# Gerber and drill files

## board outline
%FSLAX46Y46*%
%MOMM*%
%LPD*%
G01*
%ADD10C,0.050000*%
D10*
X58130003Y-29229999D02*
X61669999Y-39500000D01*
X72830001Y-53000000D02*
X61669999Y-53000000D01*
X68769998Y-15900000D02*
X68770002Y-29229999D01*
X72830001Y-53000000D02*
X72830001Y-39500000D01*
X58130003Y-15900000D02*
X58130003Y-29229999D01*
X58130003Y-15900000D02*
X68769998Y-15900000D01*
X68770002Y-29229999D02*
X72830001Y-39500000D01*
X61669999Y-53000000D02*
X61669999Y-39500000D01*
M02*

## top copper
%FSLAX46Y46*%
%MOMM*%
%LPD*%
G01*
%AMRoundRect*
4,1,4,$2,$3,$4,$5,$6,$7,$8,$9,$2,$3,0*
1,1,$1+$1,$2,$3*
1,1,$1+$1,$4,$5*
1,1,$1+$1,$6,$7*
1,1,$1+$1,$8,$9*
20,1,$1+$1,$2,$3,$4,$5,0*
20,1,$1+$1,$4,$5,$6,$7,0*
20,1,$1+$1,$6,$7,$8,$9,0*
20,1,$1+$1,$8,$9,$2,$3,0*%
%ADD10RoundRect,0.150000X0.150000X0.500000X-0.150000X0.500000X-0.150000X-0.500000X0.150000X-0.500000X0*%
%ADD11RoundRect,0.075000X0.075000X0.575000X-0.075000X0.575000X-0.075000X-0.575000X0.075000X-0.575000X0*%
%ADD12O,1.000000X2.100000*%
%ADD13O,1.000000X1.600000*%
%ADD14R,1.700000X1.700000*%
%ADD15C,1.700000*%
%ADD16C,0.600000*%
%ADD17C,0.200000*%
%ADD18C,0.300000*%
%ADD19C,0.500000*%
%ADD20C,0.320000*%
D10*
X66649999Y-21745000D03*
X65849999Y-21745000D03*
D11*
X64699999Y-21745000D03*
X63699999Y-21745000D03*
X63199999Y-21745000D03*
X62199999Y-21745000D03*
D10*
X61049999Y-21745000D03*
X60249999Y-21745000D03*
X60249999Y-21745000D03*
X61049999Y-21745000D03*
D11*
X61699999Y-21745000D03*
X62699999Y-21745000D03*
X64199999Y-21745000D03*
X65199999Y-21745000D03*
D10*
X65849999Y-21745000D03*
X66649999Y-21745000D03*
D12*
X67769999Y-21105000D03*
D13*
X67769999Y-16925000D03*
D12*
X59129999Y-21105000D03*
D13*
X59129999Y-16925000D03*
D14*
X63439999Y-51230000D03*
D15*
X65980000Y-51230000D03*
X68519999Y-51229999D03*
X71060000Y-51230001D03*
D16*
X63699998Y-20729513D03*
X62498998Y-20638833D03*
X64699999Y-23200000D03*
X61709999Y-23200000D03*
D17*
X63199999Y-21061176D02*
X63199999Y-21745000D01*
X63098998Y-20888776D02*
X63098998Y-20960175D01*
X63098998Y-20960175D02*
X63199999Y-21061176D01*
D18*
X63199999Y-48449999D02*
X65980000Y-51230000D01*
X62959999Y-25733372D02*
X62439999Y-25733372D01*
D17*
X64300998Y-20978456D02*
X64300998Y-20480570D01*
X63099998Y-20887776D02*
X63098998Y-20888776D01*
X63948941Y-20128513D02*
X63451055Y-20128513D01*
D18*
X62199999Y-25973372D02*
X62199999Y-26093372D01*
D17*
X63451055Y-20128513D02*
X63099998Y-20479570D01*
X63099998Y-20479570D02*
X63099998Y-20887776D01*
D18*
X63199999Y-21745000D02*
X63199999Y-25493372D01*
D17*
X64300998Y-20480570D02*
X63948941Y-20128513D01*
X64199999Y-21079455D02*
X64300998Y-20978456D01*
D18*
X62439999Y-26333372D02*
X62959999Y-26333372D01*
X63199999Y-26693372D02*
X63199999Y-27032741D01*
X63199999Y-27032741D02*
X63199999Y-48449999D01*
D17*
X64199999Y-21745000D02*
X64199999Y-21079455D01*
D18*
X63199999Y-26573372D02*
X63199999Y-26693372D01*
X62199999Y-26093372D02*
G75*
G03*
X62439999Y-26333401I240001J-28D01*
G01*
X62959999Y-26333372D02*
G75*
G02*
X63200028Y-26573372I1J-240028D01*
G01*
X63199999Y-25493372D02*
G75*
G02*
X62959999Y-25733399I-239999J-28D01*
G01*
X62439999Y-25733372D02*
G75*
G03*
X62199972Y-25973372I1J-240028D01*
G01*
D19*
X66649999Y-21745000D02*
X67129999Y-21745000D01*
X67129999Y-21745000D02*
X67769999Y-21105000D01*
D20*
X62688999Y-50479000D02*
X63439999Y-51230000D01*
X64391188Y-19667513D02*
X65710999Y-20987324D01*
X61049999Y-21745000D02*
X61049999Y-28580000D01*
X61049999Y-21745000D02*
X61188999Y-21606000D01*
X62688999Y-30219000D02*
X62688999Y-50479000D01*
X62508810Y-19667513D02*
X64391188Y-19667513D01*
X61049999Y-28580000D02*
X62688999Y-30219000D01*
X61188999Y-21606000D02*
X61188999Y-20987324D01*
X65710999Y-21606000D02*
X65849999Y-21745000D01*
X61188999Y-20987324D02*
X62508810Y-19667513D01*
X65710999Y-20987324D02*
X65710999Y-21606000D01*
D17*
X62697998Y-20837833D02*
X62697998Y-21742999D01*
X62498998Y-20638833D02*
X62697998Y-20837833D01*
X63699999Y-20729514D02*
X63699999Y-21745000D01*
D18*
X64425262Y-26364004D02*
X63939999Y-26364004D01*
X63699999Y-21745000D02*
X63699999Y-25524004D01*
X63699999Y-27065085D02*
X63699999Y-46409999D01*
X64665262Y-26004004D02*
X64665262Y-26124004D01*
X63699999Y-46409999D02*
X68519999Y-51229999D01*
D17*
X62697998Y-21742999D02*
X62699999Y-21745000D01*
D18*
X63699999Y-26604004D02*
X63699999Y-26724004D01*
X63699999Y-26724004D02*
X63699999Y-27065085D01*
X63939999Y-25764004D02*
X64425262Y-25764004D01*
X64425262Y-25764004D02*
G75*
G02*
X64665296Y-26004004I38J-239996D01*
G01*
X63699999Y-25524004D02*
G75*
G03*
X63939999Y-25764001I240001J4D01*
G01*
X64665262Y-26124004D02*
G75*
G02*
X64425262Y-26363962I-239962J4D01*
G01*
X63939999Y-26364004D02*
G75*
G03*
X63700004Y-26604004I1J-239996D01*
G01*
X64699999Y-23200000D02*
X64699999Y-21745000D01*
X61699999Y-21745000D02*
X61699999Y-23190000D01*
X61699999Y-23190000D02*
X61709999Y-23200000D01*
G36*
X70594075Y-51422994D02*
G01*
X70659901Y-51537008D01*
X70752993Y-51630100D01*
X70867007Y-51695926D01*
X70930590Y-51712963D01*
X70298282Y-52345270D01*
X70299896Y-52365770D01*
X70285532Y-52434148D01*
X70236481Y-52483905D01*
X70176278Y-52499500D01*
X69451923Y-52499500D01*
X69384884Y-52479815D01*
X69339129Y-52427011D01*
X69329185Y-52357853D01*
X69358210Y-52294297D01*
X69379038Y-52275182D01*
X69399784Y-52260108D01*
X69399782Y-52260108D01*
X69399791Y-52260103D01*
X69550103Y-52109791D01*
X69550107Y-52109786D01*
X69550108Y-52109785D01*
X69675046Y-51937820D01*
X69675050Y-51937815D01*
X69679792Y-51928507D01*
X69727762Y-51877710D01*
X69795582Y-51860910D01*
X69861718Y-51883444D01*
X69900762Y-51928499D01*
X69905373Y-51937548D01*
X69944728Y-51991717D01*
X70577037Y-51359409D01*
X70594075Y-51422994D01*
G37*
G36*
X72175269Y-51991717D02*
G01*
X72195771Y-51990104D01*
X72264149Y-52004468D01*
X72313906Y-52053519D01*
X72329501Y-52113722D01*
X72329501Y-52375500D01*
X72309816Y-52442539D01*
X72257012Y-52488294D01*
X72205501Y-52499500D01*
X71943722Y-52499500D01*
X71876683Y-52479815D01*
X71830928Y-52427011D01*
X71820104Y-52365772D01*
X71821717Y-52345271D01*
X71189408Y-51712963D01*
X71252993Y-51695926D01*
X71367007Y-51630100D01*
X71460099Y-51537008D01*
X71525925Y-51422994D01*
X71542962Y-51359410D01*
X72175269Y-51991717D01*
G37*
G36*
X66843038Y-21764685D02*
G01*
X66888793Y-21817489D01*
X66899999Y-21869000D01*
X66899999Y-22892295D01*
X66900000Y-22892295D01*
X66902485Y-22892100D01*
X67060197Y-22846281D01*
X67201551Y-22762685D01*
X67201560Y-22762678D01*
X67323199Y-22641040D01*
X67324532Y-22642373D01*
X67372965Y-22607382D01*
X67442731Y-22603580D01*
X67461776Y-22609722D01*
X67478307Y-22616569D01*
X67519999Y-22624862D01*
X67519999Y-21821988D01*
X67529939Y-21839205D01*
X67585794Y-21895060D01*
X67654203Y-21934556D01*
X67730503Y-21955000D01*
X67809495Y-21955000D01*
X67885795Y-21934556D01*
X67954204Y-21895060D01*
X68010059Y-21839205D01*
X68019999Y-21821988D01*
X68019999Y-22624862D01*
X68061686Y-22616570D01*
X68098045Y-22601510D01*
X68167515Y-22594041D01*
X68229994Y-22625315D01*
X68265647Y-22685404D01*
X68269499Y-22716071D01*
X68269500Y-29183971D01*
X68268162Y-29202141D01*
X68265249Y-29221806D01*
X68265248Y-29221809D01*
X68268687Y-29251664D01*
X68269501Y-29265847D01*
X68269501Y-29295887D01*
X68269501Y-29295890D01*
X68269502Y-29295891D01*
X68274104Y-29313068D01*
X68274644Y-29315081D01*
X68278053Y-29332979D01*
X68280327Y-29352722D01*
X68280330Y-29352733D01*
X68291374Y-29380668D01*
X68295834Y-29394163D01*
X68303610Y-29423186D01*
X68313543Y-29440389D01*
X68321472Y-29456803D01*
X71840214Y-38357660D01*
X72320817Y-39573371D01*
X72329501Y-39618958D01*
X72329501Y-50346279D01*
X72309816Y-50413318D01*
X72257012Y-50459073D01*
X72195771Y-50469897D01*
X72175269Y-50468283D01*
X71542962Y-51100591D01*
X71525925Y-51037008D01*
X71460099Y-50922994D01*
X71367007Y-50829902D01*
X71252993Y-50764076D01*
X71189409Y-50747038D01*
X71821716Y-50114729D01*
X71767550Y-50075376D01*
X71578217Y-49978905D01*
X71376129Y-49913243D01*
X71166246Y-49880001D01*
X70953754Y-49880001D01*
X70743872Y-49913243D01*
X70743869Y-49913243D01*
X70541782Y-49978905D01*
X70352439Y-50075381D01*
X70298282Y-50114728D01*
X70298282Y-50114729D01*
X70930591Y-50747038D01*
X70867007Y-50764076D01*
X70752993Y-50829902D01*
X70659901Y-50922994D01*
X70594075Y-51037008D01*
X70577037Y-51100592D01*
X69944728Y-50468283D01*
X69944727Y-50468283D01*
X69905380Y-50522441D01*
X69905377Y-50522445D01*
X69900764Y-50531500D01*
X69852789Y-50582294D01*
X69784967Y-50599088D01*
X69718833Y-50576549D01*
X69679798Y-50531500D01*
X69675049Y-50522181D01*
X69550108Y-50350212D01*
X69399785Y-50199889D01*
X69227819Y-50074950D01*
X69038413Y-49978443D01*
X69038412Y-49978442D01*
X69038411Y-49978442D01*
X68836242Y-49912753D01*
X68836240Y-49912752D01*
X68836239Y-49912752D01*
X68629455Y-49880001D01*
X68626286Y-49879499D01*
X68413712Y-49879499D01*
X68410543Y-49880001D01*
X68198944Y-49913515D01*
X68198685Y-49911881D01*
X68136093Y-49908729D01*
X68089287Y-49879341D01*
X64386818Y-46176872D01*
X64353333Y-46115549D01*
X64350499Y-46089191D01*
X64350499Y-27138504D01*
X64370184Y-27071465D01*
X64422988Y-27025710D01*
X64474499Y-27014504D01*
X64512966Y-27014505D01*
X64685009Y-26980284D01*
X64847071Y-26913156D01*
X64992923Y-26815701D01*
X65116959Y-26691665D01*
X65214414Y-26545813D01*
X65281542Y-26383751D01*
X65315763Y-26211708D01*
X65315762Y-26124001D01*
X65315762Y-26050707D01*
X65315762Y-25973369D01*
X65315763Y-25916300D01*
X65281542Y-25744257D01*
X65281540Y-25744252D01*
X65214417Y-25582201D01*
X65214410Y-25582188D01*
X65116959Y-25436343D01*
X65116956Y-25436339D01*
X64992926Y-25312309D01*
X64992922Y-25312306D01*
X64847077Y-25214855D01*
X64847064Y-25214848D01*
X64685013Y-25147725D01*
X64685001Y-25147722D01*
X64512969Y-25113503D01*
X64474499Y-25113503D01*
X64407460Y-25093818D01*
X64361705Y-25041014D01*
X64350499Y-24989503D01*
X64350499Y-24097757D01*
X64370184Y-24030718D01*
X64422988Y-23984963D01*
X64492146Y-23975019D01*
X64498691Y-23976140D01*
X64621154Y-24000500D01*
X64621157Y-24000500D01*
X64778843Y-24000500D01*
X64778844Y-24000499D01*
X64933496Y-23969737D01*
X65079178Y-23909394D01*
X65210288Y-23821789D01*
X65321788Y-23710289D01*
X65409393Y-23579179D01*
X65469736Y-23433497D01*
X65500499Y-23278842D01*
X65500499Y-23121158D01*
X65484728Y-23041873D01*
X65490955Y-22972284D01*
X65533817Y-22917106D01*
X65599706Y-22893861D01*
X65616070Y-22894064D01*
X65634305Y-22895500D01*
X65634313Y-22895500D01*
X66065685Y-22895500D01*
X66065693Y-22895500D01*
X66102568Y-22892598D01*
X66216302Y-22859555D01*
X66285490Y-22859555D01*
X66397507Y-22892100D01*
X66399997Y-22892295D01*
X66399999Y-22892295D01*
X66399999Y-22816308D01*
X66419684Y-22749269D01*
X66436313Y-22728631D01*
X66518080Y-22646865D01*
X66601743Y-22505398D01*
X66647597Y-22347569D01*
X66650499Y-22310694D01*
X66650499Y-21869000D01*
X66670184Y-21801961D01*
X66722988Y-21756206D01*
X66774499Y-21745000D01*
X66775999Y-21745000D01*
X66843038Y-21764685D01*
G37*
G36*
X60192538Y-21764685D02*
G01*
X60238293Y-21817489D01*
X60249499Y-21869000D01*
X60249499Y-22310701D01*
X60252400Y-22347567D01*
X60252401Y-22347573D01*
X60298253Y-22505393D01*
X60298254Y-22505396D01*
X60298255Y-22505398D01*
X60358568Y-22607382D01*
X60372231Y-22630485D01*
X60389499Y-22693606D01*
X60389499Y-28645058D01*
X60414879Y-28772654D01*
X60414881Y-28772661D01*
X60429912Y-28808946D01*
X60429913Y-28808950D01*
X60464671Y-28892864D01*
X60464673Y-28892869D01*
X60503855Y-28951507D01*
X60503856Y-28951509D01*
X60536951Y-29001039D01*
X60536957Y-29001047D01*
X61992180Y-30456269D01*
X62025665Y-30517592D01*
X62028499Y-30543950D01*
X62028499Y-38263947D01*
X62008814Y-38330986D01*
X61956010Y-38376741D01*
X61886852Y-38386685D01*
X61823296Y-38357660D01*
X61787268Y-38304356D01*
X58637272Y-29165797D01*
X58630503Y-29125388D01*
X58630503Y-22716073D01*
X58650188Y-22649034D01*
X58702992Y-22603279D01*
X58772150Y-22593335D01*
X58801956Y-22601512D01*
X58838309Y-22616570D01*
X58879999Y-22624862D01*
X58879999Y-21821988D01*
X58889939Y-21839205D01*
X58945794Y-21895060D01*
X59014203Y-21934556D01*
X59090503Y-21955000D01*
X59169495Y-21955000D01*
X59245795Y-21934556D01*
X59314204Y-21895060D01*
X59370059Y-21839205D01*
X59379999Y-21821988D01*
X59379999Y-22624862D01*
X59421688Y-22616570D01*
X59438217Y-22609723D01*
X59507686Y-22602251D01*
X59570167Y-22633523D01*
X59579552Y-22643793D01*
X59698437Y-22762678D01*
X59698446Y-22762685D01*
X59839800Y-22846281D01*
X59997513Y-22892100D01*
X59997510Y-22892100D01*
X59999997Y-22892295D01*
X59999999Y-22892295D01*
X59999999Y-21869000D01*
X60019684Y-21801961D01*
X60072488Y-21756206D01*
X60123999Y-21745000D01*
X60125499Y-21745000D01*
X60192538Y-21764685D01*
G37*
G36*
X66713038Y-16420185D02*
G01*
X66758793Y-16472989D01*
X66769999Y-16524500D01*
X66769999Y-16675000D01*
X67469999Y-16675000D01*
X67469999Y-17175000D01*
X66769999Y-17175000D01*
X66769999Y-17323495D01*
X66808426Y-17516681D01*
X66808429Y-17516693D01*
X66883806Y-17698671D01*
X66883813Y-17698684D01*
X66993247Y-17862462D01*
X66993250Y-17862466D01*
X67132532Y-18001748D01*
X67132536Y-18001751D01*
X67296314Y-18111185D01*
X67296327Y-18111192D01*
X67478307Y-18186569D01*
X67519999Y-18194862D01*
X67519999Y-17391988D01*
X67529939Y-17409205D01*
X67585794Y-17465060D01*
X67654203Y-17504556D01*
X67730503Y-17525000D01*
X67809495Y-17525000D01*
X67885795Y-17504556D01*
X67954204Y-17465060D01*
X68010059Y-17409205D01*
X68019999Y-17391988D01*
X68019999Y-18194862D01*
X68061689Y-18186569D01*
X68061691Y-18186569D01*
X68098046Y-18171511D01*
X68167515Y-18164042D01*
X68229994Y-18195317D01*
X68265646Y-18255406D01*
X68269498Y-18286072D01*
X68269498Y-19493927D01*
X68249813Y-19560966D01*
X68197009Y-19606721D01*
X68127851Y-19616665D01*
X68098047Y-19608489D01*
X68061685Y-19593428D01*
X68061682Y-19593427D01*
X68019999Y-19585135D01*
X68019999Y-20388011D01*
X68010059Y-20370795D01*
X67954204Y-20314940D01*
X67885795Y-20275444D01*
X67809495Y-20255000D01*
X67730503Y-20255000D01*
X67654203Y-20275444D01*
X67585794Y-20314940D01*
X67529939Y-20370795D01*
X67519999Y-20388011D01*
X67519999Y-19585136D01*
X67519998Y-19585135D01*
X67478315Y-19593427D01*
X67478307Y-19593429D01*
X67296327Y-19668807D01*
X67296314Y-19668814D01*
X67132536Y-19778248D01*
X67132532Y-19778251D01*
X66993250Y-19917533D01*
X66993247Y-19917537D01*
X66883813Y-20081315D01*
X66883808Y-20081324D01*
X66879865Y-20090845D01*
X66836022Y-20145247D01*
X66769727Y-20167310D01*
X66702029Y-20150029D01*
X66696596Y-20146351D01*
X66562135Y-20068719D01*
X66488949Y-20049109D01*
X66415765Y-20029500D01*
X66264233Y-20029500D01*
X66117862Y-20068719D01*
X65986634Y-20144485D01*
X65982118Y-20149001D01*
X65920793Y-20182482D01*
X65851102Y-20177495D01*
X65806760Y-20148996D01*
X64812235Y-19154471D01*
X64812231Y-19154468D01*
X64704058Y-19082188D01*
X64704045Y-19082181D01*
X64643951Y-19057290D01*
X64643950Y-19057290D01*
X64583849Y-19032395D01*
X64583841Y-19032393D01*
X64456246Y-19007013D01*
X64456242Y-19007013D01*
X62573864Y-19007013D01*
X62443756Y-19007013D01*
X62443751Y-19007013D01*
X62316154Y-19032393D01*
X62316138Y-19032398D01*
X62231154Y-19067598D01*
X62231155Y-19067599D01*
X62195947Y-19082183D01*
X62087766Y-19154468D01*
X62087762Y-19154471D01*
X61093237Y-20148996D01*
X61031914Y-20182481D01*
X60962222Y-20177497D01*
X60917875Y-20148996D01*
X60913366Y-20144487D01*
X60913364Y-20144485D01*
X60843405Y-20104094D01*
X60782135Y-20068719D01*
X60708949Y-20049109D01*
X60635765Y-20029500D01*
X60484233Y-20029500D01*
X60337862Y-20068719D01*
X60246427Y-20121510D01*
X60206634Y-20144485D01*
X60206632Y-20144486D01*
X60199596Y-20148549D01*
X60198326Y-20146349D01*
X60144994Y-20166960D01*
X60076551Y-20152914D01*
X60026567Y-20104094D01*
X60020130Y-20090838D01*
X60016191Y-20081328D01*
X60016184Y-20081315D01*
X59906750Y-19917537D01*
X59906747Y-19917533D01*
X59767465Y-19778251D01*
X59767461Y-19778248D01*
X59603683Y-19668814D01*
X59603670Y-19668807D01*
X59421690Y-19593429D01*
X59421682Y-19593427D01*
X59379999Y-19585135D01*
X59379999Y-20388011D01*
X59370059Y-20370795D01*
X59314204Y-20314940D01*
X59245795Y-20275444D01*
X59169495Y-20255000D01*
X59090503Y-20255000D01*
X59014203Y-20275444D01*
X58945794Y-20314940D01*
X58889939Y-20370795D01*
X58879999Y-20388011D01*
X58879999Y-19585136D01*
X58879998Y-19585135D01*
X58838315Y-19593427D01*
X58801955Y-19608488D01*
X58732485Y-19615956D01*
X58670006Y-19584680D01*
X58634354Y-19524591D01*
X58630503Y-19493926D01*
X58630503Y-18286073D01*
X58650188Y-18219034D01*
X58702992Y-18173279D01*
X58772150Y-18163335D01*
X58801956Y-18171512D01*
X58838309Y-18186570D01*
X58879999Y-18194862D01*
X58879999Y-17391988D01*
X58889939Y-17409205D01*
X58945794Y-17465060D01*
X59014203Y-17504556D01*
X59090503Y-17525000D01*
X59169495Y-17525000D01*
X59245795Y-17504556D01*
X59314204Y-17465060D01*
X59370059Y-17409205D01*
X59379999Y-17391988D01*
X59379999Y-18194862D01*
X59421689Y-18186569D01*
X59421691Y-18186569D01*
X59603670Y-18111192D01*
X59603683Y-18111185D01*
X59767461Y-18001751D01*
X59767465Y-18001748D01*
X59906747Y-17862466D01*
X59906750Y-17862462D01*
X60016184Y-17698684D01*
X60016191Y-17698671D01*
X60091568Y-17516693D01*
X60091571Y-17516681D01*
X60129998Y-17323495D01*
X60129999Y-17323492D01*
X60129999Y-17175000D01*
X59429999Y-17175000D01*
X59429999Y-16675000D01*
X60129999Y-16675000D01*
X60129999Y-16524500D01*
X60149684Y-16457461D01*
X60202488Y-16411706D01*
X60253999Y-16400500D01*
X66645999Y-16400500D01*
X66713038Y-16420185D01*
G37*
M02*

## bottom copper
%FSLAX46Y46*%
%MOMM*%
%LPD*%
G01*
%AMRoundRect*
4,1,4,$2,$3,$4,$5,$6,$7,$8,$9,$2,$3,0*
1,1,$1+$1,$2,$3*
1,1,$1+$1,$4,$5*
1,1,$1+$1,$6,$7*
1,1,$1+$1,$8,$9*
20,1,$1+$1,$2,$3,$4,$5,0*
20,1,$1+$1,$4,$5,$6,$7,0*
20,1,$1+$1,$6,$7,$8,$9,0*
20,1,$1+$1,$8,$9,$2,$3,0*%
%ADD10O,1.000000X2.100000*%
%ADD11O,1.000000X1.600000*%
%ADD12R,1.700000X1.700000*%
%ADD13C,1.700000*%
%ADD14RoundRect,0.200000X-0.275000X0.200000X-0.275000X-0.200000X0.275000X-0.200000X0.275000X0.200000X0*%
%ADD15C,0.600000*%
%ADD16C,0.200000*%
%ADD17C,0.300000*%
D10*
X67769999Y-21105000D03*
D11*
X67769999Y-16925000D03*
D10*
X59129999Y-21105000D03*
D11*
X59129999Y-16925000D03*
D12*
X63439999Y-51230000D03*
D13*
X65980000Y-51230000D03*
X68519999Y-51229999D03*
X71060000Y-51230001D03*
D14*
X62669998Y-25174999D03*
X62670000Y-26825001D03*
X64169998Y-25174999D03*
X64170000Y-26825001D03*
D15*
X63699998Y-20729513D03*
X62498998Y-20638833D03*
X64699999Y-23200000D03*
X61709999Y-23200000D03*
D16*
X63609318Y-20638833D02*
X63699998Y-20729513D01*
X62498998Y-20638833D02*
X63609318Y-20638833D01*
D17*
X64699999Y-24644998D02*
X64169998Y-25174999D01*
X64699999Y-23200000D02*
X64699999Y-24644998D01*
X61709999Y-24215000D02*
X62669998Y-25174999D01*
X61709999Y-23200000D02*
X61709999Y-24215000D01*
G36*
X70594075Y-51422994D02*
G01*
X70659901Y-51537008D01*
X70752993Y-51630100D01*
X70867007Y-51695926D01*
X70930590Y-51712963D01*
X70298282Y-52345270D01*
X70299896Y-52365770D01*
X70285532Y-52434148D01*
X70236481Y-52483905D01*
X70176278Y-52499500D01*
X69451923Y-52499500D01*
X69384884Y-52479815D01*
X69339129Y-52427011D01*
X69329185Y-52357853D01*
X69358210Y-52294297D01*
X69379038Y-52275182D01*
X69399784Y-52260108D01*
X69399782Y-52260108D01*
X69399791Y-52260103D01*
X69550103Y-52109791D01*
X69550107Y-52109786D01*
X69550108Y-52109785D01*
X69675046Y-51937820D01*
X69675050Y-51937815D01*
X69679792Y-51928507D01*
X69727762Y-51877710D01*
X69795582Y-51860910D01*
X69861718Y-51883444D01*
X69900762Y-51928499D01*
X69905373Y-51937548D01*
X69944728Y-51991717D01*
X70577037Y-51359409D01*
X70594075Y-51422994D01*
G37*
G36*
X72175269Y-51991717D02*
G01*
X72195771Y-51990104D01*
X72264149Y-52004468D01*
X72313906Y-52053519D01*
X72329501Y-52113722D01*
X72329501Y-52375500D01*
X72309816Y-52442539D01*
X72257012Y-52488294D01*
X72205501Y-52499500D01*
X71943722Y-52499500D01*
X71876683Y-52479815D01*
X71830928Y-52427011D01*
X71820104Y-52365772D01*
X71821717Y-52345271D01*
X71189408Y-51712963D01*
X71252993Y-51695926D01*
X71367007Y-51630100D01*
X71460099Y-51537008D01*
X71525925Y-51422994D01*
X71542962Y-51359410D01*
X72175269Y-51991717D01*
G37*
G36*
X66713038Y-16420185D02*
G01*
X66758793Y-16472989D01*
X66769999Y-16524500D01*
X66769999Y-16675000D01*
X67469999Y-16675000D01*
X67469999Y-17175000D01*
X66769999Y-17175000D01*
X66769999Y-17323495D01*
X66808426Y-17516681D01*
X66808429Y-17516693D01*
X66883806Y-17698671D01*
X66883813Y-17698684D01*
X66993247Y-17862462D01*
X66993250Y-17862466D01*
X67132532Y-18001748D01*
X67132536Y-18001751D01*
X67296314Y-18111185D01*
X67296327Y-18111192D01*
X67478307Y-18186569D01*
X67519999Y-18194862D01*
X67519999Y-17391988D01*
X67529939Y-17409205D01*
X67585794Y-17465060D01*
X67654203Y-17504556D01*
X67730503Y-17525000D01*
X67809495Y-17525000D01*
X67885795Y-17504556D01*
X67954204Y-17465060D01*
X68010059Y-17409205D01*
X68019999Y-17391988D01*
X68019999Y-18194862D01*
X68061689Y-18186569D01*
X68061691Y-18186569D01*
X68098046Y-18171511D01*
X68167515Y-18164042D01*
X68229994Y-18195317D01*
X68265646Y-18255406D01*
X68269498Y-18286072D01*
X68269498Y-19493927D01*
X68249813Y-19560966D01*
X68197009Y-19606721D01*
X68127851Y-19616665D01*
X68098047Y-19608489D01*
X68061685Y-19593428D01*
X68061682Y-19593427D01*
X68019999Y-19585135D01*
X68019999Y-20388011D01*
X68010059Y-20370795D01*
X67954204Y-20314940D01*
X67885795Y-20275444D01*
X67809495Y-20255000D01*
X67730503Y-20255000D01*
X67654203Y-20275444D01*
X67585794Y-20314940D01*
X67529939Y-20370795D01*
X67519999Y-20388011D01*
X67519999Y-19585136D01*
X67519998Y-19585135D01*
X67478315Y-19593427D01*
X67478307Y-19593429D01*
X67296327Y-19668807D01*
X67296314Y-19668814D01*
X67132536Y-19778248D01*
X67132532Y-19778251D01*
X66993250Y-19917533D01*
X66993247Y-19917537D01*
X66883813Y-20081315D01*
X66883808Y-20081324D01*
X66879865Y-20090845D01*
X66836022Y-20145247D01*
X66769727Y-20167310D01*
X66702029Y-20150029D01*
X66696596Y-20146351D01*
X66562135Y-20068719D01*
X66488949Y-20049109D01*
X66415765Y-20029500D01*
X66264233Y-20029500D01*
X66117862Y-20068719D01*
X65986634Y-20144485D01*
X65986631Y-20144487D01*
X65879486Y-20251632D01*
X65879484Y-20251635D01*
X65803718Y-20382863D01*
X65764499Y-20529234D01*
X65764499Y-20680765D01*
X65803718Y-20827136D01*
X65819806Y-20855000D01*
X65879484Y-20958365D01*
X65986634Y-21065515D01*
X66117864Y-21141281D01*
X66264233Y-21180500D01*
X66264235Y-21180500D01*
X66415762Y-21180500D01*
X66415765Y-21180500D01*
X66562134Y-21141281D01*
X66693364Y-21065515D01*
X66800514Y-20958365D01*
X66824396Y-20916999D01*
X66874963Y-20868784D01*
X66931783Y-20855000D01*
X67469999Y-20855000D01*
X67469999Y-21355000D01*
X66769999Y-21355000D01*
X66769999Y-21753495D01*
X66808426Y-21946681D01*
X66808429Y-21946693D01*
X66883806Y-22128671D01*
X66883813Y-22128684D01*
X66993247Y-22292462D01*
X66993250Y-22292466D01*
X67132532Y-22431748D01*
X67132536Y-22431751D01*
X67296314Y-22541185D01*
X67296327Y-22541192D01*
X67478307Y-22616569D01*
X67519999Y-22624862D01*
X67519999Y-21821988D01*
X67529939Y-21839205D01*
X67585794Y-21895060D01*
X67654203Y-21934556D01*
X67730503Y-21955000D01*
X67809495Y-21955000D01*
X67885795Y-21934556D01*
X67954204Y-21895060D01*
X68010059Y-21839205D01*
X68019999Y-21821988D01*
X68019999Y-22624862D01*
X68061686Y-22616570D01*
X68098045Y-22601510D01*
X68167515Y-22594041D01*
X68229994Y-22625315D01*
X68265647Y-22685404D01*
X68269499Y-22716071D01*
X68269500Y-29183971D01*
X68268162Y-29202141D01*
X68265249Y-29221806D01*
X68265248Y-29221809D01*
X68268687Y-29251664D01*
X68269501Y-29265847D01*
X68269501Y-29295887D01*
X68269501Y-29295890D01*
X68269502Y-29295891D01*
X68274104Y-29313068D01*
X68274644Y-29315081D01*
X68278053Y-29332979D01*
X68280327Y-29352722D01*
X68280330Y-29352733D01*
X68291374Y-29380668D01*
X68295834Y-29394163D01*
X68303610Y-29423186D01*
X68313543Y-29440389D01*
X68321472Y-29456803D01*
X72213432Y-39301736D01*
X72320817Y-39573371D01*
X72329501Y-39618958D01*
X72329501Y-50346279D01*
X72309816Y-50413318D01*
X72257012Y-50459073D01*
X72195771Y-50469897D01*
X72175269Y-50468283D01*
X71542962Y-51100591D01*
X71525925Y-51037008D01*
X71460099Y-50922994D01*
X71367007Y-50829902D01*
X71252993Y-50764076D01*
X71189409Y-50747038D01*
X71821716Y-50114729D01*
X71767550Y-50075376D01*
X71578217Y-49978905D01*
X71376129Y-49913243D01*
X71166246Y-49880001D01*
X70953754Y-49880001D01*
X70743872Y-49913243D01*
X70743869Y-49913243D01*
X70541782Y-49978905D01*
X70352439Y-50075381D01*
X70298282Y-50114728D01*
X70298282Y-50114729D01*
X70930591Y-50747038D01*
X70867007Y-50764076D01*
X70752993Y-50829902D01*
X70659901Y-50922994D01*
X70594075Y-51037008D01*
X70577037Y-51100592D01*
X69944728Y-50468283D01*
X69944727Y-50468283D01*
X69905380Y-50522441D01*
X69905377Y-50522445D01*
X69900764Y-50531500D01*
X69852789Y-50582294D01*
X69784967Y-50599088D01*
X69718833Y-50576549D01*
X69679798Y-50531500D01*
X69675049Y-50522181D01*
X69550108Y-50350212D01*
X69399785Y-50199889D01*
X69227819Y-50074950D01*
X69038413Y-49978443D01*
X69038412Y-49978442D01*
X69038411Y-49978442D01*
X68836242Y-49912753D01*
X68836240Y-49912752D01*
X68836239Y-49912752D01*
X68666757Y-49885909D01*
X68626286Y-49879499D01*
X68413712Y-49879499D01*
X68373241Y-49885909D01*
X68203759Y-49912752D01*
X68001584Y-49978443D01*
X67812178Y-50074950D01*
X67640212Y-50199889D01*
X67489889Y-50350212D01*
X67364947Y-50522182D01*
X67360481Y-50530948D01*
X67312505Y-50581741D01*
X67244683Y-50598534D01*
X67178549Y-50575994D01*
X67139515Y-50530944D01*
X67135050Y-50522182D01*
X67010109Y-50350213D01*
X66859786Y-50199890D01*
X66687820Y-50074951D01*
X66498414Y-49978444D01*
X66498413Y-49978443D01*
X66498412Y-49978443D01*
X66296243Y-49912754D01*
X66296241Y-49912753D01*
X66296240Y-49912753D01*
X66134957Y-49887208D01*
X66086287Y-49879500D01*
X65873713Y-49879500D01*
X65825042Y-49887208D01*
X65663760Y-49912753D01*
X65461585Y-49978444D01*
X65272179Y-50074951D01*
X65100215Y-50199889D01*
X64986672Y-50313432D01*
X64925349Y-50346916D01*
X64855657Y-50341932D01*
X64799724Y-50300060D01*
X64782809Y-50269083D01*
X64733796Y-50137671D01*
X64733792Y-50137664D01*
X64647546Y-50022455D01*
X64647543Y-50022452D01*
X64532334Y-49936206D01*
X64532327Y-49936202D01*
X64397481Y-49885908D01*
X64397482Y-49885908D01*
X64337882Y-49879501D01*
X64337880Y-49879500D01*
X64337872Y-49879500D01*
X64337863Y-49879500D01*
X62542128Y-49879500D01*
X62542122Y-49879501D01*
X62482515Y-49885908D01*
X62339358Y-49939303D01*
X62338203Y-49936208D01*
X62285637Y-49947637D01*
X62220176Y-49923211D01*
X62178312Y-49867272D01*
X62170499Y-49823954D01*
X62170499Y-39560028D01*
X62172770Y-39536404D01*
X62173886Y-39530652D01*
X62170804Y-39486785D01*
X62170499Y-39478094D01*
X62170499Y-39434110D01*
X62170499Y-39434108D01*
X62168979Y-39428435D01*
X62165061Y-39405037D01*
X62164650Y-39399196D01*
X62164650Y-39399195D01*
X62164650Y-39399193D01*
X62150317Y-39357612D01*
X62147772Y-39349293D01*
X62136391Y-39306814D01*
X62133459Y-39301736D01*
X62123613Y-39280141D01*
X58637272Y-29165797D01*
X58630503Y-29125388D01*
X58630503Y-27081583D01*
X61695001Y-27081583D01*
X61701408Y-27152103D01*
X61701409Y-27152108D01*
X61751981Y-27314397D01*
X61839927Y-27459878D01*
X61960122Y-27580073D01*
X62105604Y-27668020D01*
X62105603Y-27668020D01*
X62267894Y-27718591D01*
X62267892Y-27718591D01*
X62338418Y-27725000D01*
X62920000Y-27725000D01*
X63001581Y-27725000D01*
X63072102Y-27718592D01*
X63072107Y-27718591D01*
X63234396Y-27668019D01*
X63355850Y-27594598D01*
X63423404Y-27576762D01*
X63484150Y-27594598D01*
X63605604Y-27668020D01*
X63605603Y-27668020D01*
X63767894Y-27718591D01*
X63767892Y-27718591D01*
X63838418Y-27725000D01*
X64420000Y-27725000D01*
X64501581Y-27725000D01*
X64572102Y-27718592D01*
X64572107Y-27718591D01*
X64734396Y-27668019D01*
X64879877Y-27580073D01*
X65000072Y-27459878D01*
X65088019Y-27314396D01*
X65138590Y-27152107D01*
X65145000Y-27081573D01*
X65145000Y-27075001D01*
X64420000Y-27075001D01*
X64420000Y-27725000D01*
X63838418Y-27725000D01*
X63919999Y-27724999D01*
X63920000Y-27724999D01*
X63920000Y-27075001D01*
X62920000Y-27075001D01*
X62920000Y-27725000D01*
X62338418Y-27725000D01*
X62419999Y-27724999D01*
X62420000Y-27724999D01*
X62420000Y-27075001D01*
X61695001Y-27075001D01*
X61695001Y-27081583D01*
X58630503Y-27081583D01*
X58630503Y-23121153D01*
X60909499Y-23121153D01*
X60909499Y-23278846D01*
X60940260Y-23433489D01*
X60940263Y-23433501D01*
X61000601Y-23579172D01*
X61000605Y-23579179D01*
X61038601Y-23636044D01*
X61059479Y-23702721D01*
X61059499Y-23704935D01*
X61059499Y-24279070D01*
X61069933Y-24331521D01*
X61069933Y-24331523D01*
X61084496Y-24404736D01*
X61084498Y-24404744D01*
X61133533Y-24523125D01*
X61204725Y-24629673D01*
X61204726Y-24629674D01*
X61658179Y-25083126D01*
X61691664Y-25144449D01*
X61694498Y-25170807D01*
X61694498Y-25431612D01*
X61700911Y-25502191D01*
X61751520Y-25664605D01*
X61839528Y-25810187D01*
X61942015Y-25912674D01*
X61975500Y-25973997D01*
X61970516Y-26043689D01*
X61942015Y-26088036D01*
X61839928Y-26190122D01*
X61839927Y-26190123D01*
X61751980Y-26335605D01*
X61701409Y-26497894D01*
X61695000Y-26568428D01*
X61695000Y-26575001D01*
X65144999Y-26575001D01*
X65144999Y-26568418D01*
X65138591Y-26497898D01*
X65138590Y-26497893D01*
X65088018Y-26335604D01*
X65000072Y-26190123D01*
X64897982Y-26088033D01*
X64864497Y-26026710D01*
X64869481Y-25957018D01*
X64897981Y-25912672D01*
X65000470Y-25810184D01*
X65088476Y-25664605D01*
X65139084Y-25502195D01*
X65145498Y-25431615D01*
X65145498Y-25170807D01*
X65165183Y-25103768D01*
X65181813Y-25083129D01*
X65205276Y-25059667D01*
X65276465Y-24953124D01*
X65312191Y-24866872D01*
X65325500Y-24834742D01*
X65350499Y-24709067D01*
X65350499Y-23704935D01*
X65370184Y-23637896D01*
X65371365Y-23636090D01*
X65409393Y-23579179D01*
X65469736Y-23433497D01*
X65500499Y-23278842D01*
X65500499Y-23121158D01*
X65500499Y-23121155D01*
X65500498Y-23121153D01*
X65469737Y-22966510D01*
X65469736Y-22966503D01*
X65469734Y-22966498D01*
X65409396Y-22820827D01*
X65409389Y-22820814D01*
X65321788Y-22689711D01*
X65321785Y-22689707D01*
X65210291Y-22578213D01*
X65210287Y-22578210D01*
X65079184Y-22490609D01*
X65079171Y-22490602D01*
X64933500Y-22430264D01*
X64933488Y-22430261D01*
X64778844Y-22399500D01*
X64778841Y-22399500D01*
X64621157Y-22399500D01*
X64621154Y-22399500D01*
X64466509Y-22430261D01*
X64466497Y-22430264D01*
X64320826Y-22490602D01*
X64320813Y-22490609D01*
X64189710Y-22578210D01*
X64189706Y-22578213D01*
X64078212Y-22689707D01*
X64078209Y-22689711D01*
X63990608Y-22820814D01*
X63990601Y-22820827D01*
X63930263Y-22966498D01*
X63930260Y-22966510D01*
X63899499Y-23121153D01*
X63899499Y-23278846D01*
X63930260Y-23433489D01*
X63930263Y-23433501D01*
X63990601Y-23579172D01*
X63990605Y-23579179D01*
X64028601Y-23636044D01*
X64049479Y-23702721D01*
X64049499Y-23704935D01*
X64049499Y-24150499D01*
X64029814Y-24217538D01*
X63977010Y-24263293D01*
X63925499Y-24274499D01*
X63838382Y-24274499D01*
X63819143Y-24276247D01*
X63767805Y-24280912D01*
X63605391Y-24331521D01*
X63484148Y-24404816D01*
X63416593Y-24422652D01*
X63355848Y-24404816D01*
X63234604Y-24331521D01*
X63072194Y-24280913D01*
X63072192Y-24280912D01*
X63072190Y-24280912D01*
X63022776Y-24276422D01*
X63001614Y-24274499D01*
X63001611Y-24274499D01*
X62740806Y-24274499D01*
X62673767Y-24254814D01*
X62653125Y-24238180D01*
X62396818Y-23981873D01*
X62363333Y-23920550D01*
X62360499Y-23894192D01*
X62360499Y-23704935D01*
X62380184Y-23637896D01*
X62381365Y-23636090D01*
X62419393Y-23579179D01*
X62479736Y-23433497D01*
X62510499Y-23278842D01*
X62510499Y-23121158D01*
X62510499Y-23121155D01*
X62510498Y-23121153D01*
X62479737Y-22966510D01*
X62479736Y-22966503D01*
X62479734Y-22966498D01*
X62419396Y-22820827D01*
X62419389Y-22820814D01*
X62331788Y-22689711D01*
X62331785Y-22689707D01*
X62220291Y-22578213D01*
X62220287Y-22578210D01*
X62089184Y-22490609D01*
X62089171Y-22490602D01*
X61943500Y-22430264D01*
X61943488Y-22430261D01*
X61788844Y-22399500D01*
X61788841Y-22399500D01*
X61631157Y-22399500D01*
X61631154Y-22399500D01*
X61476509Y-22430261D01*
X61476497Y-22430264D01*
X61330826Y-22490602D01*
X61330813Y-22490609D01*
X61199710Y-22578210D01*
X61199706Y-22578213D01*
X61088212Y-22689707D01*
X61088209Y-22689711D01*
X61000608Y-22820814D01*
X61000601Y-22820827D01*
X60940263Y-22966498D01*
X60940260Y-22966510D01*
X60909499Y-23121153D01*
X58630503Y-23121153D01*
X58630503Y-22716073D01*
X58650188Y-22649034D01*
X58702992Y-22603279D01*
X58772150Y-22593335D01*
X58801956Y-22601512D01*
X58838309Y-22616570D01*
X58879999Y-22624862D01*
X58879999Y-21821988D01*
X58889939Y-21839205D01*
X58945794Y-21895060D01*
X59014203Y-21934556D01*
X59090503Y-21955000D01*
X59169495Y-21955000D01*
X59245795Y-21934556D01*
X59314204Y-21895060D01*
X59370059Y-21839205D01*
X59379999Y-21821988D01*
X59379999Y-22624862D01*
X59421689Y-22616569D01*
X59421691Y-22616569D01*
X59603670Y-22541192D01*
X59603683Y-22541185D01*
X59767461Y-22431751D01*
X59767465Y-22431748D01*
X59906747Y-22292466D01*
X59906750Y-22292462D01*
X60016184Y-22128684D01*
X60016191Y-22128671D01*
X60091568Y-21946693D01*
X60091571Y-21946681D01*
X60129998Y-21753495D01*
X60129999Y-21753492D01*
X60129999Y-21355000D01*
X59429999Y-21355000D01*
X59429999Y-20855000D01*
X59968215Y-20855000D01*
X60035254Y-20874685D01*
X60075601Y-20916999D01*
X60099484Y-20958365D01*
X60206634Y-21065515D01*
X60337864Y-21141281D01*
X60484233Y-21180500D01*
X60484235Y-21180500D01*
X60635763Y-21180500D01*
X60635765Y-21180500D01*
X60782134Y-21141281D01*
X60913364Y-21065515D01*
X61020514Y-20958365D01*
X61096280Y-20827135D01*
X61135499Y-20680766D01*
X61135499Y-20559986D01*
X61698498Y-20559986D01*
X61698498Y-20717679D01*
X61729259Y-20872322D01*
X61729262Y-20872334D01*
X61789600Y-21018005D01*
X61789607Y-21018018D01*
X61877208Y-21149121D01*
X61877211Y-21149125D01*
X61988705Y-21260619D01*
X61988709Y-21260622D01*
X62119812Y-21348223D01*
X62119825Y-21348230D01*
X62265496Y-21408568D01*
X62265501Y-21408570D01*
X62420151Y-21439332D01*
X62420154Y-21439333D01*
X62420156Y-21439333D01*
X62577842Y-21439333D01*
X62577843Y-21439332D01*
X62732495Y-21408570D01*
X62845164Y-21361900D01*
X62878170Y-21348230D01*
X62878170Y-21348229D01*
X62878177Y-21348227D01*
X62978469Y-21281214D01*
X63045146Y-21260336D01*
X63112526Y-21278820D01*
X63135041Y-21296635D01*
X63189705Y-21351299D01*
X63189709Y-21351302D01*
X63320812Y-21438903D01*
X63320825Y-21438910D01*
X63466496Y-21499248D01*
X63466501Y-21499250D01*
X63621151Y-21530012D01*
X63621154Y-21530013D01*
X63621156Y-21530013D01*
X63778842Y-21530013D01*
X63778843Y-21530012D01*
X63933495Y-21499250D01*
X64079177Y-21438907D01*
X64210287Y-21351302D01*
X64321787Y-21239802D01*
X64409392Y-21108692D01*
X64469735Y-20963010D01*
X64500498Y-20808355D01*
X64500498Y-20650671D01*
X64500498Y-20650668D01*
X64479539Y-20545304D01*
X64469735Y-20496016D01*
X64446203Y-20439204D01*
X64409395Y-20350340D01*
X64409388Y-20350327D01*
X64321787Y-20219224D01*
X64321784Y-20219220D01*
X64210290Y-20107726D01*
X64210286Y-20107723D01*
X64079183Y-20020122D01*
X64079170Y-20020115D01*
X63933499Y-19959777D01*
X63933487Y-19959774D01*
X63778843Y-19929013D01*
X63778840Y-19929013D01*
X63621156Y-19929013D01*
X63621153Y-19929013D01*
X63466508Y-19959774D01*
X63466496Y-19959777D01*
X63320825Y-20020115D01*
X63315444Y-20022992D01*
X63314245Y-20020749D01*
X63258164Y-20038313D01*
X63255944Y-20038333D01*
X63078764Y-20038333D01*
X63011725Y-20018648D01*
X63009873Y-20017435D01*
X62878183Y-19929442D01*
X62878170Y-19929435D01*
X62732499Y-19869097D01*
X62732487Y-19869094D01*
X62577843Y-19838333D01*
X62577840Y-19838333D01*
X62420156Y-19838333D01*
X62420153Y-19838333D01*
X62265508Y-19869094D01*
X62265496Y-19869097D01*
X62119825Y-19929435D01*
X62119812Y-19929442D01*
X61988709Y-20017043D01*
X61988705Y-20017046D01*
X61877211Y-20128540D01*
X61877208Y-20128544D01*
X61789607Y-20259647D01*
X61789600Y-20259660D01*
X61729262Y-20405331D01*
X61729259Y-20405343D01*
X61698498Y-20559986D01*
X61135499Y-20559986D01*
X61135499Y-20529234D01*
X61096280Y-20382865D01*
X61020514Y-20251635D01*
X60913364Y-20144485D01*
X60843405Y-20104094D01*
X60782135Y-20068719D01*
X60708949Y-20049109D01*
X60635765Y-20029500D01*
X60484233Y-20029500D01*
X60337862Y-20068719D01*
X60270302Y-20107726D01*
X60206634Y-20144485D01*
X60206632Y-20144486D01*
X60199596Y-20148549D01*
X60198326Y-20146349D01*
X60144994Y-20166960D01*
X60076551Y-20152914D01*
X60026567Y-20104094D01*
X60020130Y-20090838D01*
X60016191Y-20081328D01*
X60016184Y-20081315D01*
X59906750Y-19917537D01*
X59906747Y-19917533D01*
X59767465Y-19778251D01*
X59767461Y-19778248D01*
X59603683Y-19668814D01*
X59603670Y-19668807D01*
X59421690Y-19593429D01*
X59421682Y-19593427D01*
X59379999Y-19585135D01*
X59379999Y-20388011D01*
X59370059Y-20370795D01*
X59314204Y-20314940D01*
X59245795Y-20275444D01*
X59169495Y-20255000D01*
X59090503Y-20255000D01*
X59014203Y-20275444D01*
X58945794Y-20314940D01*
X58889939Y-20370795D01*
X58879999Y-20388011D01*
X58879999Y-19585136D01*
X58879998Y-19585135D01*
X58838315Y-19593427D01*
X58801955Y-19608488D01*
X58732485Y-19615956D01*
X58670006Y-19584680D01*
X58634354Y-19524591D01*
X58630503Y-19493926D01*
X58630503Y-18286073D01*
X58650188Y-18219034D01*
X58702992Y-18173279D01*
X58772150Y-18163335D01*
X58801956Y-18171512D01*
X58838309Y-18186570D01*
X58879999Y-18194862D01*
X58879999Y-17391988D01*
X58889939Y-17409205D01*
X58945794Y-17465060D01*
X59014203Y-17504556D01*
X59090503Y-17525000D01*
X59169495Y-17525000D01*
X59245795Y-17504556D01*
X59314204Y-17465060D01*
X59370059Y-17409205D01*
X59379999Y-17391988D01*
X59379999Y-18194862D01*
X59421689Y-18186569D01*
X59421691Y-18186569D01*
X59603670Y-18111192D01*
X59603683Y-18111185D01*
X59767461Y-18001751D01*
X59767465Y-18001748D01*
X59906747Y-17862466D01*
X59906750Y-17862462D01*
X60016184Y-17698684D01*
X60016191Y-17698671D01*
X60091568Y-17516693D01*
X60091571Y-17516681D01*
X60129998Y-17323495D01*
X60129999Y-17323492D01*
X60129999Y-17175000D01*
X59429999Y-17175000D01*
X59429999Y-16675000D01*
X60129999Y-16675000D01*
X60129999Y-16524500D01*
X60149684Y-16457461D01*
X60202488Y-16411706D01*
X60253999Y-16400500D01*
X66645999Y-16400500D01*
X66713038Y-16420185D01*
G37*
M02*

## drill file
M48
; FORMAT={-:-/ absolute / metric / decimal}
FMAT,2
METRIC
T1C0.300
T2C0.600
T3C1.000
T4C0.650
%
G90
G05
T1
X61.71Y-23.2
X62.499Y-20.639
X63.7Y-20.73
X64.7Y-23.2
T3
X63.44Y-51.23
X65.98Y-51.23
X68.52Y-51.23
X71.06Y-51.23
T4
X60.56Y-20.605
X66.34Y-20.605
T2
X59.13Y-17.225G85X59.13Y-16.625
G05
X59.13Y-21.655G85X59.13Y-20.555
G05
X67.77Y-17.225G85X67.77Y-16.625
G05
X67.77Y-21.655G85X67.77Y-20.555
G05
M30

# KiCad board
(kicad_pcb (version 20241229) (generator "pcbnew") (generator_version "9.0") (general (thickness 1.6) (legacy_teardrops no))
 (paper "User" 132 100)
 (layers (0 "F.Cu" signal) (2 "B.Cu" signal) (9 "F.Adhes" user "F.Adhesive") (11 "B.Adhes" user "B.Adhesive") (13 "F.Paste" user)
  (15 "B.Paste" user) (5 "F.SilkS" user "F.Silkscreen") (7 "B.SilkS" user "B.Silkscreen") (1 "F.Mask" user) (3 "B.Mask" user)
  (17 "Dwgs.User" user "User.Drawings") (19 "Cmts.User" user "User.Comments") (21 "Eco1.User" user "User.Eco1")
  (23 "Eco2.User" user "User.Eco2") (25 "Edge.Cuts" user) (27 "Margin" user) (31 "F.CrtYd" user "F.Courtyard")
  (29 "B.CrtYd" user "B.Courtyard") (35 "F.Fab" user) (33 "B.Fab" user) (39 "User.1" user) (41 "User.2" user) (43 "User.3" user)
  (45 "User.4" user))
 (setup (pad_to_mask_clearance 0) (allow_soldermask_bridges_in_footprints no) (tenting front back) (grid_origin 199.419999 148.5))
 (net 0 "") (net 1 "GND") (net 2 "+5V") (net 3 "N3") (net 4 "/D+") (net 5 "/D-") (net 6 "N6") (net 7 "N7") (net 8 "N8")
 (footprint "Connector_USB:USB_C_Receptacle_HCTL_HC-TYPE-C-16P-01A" (layer "F.Cu") (at 63.449999 18 180)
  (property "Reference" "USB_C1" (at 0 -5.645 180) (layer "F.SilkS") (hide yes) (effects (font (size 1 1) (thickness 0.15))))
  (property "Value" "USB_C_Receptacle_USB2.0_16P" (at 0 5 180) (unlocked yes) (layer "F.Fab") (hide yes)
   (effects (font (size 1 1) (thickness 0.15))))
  (pad "" np_thru_hole circle (at -2.89 -2.605 180) (size 0.65 0.65) (drill 0.65) (layers "*.Mask"))
  (pad "" np_thru_hole circle (at 2.89 -2.605 180) (size 0.65 0.65) (drill 0.65) (layers "*.Mask"))
  (pad "A1" smd roundrect (at -3.2 -3.745 180) (size 0.6 1.3) (layers "F.Cu" "F.Mask" "F.Paste") (roundrect_rratio 0.25) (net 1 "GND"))
  (pad "A4" smd roundrect (at -2.4 -3.745 180) (size 0.6 1.3) (layers "F.Cu" "F.Mask" "F.Paste") (roundrect_rratio 0.25) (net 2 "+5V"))
  (pad "A5" smd roundrect (at -1.25 -3.745 180) (size 0.3 1.3) (layers "F.Cu" "F.Mask" "F.Paste") (roundrect_rratio 0.25) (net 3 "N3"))
  (pad "A6" smd roundrect (at -0.25 -3.745 180) (size 0.3 1.3) (layers "F.Cu" "F.Mask" "F.Paste") (roundrect_rratio 0.25) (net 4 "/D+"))
  (pad "A7" smd roundrect (at 0.25 -3.745 180) (size 0.3 1.3) (layers "F.Cu" "F.Mask" "F.Paste") (roundrect_rratio 0.25) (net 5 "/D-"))
  (pad "A8" smd roundrect (at 1.25 -3.745 180) (size 0.3 1.3) (layers "F.Cu" "F.Mask" "F.Paste") (roundrect_rratio 0.25) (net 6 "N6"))
  (pad "A9" smd roundrect (at 2.4 -3.745 180) (size 0.6 1.3) (layers "F.Cu" "F.Mask" "F.Paste") (roundrect_rratio 0.25) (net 2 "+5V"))
  (pad "A12" smd roundrect (at 3.2 -3.745 180) (size 0.6 1.3) (layers "F.Cu" "F.Mask" "F.Paste") (roundrect_rratio 0.25) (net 1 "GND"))
  (pad "B1" smd roundrect (at 3.2 -3.745 180) (size 0.6 1.3) (layers "F.Cu" "F.Mask" "F.Paste") (roundrect_rratio 0.25) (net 1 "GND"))
  (pad "B4" smd roundrect (at 2.4 -3.745 180) (size 0.6 1.3) (layers "F.Cu" "F.Mask" "F.Paste") (roundrect_rratio 0.25) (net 2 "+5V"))
  (pad "B5" smd roundrect (at 1.75 -3.745 180) (size 0.3 1.3) (layers "F.Cu" "F.Mask" "F.Paste") (roundrect_rratio 0.25) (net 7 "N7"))
  (pad "B6" smd roundrect (at 0.75 -3.745 180) (size 0.3 1.3) (layers "F.Cu" "F.Mask" "F.Paste") (roundrect_rratio 0.25) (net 4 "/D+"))
  (pad "B7" smd roundrect (at -0.75 -3.745 180) (size 0.3 1.3) (layers "F.Cu" "F.Mask" "F.Paste") (roundrect_rratio 0.25) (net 5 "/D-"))
  (pad "B8" smd roundrect (at -1.75 -3.745 180) (size 0.3 1.3) (layers "F.Cu" "F.Mask" "F.Paste") (roundrect_rratio 0.25) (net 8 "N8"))
  (pad "B9" smd roundrect (at -2.4 -3.745 180) (size 0.6 1.3) (layers "F.Cu" "F.Mask" "F.Paste") (roundrect_rratio 0.25) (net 2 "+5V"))
  (pad "B12" smd roundrect (at -3.2 -3.745 180) (size 0.6 1.3) (layers "F.Cu" "F.Mask" "F.Paste") (roundrect_rratio 0.25) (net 1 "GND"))
  (pad "S1" thru_hole oval (at -4.32 -3.105 180) (size 1 2.1) (drill oval 0.6 1.7) (layers "*.Cu" "*.Mask") (remove_unused_layers no)
   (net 1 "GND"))
  (pad "S1" thru_hole oval (at -4.32 1.075 180) (size 1 1.6) (drill oval 0.6 1.2) (layers "*.Cu" "*.Mask") (remove_unused_layers no)
   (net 1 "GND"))
  (pad "S1" thru_hole oval (at 4.32 -3.105 180) (size 1 2.1) (drill oval 0.6 1.7) (layers "*.Cu" "*.Mask") (remove_unused_layers no)
   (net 1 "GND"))
  (pad "S1" thru_hole oval (at 4.32 1.075 180) (size 1 1.6) (drill oval 0.6 1.2) (layers "*.Cu" "*.Mask") (remove_unused_layers no)
   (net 1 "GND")))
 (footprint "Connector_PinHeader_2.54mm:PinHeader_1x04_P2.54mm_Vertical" (layer "F.Cu") (at 63.439999 51.23 90)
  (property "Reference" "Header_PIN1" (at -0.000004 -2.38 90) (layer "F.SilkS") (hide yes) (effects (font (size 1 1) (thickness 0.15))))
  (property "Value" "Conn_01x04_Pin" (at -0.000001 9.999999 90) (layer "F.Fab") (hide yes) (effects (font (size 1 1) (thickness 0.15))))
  (pad "1" thru_hole rect (at 0 0 90) (size 1.7 1.7) (drill 1) (layers "*.Cu" "*.Mask") (remove_unused_layers no) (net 2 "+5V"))
  (pad "2" thru_hole circle (at 0 2.540001 90) (size 1.7 1.7) (drill 1) (layers "*.Cu" "*.Mask") (remove_unused_layers no) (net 5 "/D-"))
  (pad "3" thru_hole circle (at 0.000001 5.08 90) (size 1.7 1.7) (drill 1) (layers "*.Cu" "*.Mask") (remove_unused_layers no) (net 4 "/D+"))
  (pad "4" thru_hole circle (at -0.000001 7.620001 90) (size 1.7 1.7) (drill 1) (layers "*.Cu" "*.Mask") (remove_unused_layers no)
   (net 1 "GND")))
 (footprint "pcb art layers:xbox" (layer "F.Cu") (at 65.419999 34.5)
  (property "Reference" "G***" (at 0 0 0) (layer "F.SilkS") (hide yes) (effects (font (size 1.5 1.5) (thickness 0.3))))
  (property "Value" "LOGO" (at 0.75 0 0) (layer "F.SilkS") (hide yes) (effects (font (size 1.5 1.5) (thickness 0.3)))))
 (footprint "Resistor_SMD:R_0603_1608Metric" (layer "B.Cu") (at 62.669999 26 -90)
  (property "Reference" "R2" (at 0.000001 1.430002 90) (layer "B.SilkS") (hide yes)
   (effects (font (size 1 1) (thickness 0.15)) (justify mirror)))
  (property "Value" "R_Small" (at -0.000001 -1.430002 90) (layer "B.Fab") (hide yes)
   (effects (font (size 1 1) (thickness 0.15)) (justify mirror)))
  (pad "1" smd roundrect (at -0.825001 0.000001 270) (size 0.8 0.95) (layers "B.Cu" "B.Mask" "B.Paste") (roundrect_rratio 0.25) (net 7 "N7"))
  (pad "2" smd roundrect (at 0.825001 -0.000001 270) (size 0.8 0.95) (layers "B.Cu" "B.Mask" "B.Paste") (roundrect_rratio 0.25)
   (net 1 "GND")))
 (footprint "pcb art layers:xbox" (layer "B.Cu") (at 65.419999 34.5 180)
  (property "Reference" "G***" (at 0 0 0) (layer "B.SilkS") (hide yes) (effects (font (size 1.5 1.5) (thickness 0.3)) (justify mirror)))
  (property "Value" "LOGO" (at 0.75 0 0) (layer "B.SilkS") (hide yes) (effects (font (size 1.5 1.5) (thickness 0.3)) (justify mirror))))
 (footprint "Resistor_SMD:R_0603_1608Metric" (layer "B.Cu") (at 64.169999 26 -90)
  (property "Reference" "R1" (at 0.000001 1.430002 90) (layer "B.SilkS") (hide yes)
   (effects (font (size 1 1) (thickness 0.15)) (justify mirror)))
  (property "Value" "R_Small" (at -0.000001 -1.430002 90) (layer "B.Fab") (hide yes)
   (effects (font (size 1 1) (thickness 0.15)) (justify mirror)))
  (pad "1" smd roundrect (at -0.825001 0.000001 270) (size 0.8 0.95) (layers "B.Cu" "B.Mask" "B.Paste") (roundrect_rratio 0.25) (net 3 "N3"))
  (pad "2" smd roundrect (at 0.825001 -0.000001 270) (size 0.8 0.95) (layers "B.Cu" "B.Mask" "B.Paste") (roundrect_rratio 0.25)
   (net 1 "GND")))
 (gr_line (start 58.130003 29.229999) (end 61.669999 39.5) (stroke (width 0.05) (type default)) (layer "Edge.Cuts"))
 (gr_line (start 72.830001 53) (end 61.669999 53) (stroke (width 0.05) (type default)) (layer "Edge.Cuts"))
 (gr_line (start 68.769998 15.9) (end 68.770002 29.229999) (stroke (width 0.05) (type default)) (layer "Edge.Cuts"))
 (gr_line (start 72.830001 53) (end 72.830001 39.5) (stroke (width 0.05) (type default)) (layer "Edge.Cuts"))
 (gr_line (start 58.130003 15.9) (end 58.130003 29.229999) (stroke (width 0.05) (type default)) (layer "Edge.Cuts"))
 (gr_line (start 58.130003 15.9) (end 68.769998 15.9) (stroke (width 0.05) (type default)) (layer "Edge.Cuts"))
 (gr_line (start 68.770002 29.229999) (end 72.830001 39.5) (stroke (width 0.05) (type default)) (layer "Edge.Cuts"))
 (gr_line (start 61.669999 53) (end 61.669999 39.5) (stroke (width 0.05) (type default)) (layer "Edge.Cuts"))
 (segment (start 63.199999 21.061176) (end 63.199999 21.745) (width 0.2) (layer "F.Cu") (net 5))
 (segment (start 63.098998 20.888776) (end 63.098998 20.960175) (width 0.2) (layer "F.Cu") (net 5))
 (segment (start 63.098998 20.960175) (end 63.199999 21.061176) (width 0.2) (layer "F.Cu") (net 5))
 (segment (start 63.199999 48.449999) (end 65.98 51.23) (width 0.3) (layer "F.Cu") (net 5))
 (segment (start 62.959999 25.733372) (end 62.439999 25.733372) (width 0.3) (layer "F.Cu") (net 5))
 (segment (start 64.300998 20.978456) (end 64.300998 20.48057) (width 0.2) (layer "F.Cu") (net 5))
 (segment (start 63.099998 20.887776) (end 63.098998 20.888776) (width 0.2) (layer "F.Cu") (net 5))
 (segment (start 63.948941 20.128513) (end 63.451055 20.128513) (width 0.2) (layer "F.Cu") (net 5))
 (segment (start 62.199999 25.973372) (end 62.199999 26.093372) (width 0.3) (layer "F.Cu") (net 5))
 (segment (start 63.451055 20.128513) (end 63.099998 20.47957) (width 0.2) (layer "F.Cu") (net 5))
 (segment (start 63.099998 20.47957) (end 63.099998 20.887776) (width 0.2) (layer "F.Cu") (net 5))
 (segment (start 63.199999 21.745) (end 63.199999 25.493372) (width 0.3) (layer "F.Cu") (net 5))
 (segment (start 64.300998 20.48057) (end 63.948941 20.128513) (width 0.2) (layer "F.Cu") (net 5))
 (segment (start 64.199999 21.079455) (end 64.300998 20.978456) (width 0.2) (layer "F.Cu") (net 5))
 (segment (start 62.439999 26.333372) (end 62.959999 26.333372) (width 0.3) (layer "F.Cu") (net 5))
 (segment (start 63.199999 26.693372) (end 63.199999 27.032741) (width 0.3) (layer "F.Cu") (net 5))
 (segment (start 63.199999 27.032741) (end 63.199999 48.449999) (width 0.3) (layer "F.Cu") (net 5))
 (segment (start 64.199999 21.745) (end 64.199999 21.079455) (width 0.2) (layer "F.Cu") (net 5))
 (segment (start 63.199999 26.573372) (end 63.199999 26.693372) (width 0.3) (layer "F.Cu") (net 5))
 (arc (start 62.199999 26.093372) (mid 62.270293 26.263078) (end 62.439999 26.333372) (width 0.3) (layer "F.Cu") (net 5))
 (arc (start 62.959999 26.333372) (mid 63.129705 26.403666) (end 63.199999 26.573372) (width 0.3) (layer "F.Cu") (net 5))
 (arc (start 63.199999 25.493372) (mid 63.129705 25.663078) (end 62.959999 25.733372) (width 0.3) (layer "F.Cu") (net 5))
 (arc (start 62.439999 25.733372) (mid 62.270293 25.803666) (end 62.199999 25.973372) (width 0.3) (layer "F.Cu") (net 5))
 (segment (start 66.649999 21.745) (end 67.129999 21.745) (width 0.5) (layer "F.Cu") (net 1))
 (segment (start 67.129999 21.745) (end 67.769999 21.105) (width 0.5) (layer "F.Cu") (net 1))
 (segment (start 62.688999 50.479) (end 63.439999 51.23) (width 0.32) (layer "F.Cu") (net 2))
 (segment (start 64.391188 19.667513) (end 65.710999 20.987324) (width 0.32) (layer "F.Cu") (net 2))
 (segment (start 61.049999 21.745) (end 61.049999 28.58) (width 0.32) (layer "F.Cu") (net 2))
 (segment (start 61.049999 21.745) (end 61.188999 21.606) (width 0.32) (layer "F.Cu") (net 2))
 (segment (start 62.688999 30.219) (end 62.688999 50.479) (width 0.32) (layer "F.Cu") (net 2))
 (segment (start 62.50881 19.667513) (end 64.391188 19.667513) (width 0.32) (layer "F.Cu") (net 2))
 (segment (start 61.049999 28.58) (end 62.688999 30.219) (width 0.32) (layer "F.Cu") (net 2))
 (segment (start 61.188999 21.606) (end 61.188999 20.987324) (width 0.32) (layer "F.Cu") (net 2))
 (segment (start 65.710999 21.606) (end 65.849999 21.745) (width 0.32) (layer "F.Cu") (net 2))
 (segment (start 61.188999 20.987324) (end 62.50881 19.667513) (width 0.32) (layer "F.Cu") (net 2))
 (segment (start 65.710999 20.987324) (end 65.710999 21.606) (width 0.32) (layer "F.Cu") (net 2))
 (segment (start 62.697998 20.837833) (end 62.697998 21.742999) (width 0.2) (layer "F.Cu") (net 4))
 (segment (start 62.498998 20.638833) (end 62.697998 20.837833) (width 0.2) (layer "F.Cu") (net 4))
 (segment (start 63.699999 20.729514) (end 63.699999 21.745) (width 0.2) (layer "F.Cu") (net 4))
 (segment (start 64.425262 26.364004) (end 63.939999 26.364004) (width 0.3) (layer "F.Cu") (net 4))
 (segment (start 63.699999 21.745) (end 63.699999 25.524004) (width 0.3) (layer "F.Cu") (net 4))
 (segment (start 63.699999 27.065085) (end 63.699999 46.409999) (width 0.3) (layer "F.Cu") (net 4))
 (segment (start 64.665262 26.004004) (end 64.665262 26.124004) (width 0.3) (layer "F.Cu") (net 4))
 (segment (start 63.699999 46.409999) (end 68.519999 51.229999) (width 0.3) (layer "F.Cu") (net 4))
 (segment (start 62.697998 21.742999) (end 62.699999 21.745) (width 0.2) (layer "F.Cu") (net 4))
 (segment (start 63.699999 26.604004) (end 63.699999 26.724004) (width 0.3) (layer "F.Cu") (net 4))
 (segment (start 63.699999 26.724004) (end 63.699999 27.065085) (width 0.3) (layer "F.Cu") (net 4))
 (segment (start 63.939999 25.764004) (end 64.425262 25.764004) (width 0.3) (layer "F.Cu") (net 4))
 (via (at 63.699998 20.729513) (size 0.6) (drill 0.3) (layers "F.Cu" "B.Cu") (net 4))
 (via (at 62.498998 20.638833) (size 0.6) (drill 0.3) (layers "F.Cu" "B.Cu") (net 4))
 (arc (start 64.425262 25.764004) (mid 64.594968 25.834298) (end 64.665262 26.004004) (width 0.3) (layer "F.Cu") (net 4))
 (arc (start 63.699999 25.524004) (mid 63.770293 25.69371) (end 63.939999 25.764004) (width 0.3) (layer "F.Cu") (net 4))
 (arc (start 64.665262 26.124004) (mid 64.594968 26.29371) (end 64.425262 26.364004) (width 0.3) (layer "F.Cu") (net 4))
 (arc (start 63.939999 26.364004) (mid 63.770293 26.434298) (end 63.699999 26.604004) (width 0.3) (layer "F.Cu") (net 4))
 (segment (start 63.609318 20.638833) (end 63.699998 20.729513) (width 0.2) (layer "B.Cu") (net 4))
 (segment (start 62.498998 20.638833) (end 63.609318 20.638833) (width 0.2) (layer "B.Cu") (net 4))
 (segment (start 64.699999 23.2) (end 64.699999 21.745) (width 0.3) (layer "F.Cu") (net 3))
 (via (at 64.699999 23.2) (size 0.6) (drill 0.3) (layers "F.Cu" "B.Cu") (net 3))
 (segment (start 64.699999 24.644998) (end 64.169998 25.174999) (width 0.3) (layer "B.Cu") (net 3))
 (segment (start 64.699999 23.2) (end 64.699999 24.644998) (width 0.3) (layer "B.Cu") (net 3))
 (segment (start 61.699999 21.745) (end 61.699999 23.19) (width 0.3) (layer "F.Cu") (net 7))
 (segment (start 61.699999 23.19) (end 61.709999 23.2) (width 0.3) (layer "F.Cu") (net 7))
 (via (at 61.709999 23.2) (size 0.6) (drill 0.3) (layers "F.Cu" "B.Cu") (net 7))
 (segment (start 61.709999 24.215) (end 62.669998 25.174999) (width 0.3) (layer "B.Cu") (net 7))
 (segment (start 61.709999 23.2) (end 61.709999 24.215) (width 0.3) (layer "B.Cu") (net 7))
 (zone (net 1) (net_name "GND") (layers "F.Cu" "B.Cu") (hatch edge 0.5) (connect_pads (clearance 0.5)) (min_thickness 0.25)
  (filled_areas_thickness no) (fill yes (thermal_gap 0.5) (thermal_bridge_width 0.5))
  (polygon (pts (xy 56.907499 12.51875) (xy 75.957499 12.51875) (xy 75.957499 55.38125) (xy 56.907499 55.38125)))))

